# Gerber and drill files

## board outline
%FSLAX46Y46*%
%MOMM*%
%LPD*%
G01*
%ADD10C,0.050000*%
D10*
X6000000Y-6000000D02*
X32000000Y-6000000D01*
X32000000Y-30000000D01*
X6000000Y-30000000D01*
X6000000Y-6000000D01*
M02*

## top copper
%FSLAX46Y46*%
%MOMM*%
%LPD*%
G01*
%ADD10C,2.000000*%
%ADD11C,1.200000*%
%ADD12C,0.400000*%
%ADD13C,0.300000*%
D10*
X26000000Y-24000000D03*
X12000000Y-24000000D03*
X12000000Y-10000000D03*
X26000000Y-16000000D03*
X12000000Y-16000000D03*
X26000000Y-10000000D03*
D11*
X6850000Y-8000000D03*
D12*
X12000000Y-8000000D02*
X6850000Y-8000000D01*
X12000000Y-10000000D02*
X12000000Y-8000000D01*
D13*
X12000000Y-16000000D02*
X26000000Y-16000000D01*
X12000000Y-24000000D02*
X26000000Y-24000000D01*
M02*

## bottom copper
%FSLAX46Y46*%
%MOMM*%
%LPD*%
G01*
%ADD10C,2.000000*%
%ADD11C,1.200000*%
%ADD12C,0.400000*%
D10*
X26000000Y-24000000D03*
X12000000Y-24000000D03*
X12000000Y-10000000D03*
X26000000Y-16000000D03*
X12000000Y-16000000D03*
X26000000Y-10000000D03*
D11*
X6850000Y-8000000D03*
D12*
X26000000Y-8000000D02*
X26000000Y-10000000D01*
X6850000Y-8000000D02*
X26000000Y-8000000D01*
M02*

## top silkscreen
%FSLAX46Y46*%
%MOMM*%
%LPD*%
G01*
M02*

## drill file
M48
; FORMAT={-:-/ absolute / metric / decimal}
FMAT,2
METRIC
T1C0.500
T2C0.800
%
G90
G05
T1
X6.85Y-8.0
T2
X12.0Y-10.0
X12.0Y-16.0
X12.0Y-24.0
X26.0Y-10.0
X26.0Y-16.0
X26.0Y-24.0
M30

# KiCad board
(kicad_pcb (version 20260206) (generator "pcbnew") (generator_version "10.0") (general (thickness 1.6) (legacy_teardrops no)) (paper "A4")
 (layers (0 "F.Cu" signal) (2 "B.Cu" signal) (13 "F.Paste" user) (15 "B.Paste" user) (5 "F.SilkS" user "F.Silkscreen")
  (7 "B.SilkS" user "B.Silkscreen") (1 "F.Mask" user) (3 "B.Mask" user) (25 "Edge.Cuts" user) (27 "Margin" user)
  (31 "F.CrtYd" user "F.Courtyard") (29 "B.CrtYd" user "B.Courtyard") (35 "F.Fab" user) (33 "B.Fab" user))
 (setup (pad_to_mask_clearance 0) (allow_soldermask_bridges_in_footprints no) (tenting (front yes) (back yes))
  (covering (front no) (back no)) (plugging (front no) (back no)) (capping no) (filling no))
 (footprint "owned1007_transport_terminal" (layer "F.Cu") (at 26 24)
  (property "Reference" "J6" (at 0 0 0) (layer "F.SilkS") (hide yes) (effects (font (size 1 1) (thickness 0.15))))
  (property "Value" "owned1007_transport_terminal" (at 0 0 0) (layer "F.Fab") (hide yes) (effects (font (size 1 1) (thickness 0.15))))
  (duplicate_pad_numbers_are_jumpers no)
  (pad "1" thru_hole circle (at 0 0) (size 2 2) (drill 0.8) (layers "*.Cu" "*.Mask") (remove_unused_layers no) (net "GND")))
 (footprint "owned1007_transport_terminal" (layer "F.Cu") (at 12 24)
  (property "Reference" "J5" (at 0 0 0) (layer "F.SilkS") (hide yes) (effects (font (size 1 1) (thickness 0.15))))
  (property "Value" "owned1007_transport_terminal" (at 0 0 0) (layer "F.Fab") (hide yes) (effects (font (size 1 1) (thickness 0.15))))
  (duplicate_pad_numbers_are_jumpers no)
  (pad "1" thru_hole circle (at 0 0) (size 2 2) (drill 0.8) (layers "*.Cu" "*.Mask") (remove_unused_layers no) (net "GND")))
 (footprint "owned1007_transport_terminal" (layer "F.Cu") (at 12 10)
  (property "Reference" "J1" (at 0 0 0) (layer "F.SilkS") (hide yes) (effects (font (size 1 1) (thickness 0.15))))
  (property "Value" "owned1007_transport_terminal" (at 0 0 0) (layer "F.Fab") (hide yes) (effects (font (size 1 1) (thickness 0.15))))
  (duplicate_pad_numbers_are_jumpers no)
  (pad "1" thru_hole circle (at 0 0) (size 2 2) (drill 0.8) (layers "*.Cu" "*.Mask") (remove_unused_layers no) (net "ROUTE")))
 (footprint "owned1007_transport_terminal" (layer "F.Cu") (at 26 16)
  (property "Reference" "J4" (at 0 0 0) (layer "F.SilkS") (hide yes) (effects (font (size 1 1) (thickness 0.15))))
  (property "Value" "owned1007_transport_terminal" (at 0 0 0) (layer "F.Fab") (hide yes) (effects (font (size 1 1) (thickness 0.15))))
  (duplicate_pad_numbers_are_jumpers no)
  (pad "1" thru_hole circle (at 0 0) (size 2 2) (drill 0.8) (layers "*.Cu" "*.Mask") (remove_unused_layers no) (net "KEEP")))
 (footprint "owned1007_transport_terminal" (layer "F.Cu") (at 12 16)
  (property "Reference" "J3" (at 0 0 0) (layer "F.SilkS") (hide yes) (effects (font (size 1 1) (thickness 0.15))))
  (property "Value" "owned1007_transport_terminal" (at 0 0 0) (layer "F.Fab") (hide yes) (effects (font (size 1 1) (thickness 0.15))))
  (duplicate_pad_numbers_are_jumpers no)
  (pad "1" thru_hole circle (at 0 0) (size 2 2) (drill 0.8) (layers "*.Cu" "*.Mask") (remove_unused_layers no) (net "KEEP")))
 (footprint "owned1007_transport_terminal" (layer "F.Cu") (at 26 10)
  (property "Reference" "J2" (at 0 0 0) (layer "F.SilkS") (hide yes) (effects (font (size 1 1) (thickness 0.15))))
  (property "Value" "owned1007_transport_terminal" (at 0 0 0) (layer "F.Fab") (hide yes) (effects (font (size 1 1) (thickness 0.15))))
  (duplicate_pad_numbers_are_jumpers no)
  (pad "1" thru_hole circle (at 0 0) (size 2 2) (drill 0.8) (layers "*.Cu" "*.Mask") (remove_unused_layers no) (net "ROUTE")))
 (gr_rect (start 6 6) (end 32 30) (stroke (width 0.05) (type default)) (fill no) (layer "Edge.Cuts"))
 (segment (start 12 8) (end 6.85 8) (width 0.4) (layer "F.Cu") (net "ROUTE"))
 (segment (start 12 10) (end 12 8) (width 0.4) (layer "F.Cu") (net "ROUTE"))
 (via (at 6.85 8) (size 1.2) (drill 0.5) (layers "F.Cu" "B.Cu") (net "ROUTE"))
 (segment (start 26 8) (end 26 10) (width 0.4) (layer "B.Cu") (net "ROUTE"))
 (segment (start 6.85 8) (end 26 8) (width 0.4) (layer "B.Cu") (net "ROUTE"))
 (segment (start 12 16) (end 26 16) (width 0.3) (locked yes) (layer "F.Cu") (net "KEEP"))
 (segment (start 12 24) (end 26 24) (width 0.3) (layer "F.Cu") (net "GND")))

